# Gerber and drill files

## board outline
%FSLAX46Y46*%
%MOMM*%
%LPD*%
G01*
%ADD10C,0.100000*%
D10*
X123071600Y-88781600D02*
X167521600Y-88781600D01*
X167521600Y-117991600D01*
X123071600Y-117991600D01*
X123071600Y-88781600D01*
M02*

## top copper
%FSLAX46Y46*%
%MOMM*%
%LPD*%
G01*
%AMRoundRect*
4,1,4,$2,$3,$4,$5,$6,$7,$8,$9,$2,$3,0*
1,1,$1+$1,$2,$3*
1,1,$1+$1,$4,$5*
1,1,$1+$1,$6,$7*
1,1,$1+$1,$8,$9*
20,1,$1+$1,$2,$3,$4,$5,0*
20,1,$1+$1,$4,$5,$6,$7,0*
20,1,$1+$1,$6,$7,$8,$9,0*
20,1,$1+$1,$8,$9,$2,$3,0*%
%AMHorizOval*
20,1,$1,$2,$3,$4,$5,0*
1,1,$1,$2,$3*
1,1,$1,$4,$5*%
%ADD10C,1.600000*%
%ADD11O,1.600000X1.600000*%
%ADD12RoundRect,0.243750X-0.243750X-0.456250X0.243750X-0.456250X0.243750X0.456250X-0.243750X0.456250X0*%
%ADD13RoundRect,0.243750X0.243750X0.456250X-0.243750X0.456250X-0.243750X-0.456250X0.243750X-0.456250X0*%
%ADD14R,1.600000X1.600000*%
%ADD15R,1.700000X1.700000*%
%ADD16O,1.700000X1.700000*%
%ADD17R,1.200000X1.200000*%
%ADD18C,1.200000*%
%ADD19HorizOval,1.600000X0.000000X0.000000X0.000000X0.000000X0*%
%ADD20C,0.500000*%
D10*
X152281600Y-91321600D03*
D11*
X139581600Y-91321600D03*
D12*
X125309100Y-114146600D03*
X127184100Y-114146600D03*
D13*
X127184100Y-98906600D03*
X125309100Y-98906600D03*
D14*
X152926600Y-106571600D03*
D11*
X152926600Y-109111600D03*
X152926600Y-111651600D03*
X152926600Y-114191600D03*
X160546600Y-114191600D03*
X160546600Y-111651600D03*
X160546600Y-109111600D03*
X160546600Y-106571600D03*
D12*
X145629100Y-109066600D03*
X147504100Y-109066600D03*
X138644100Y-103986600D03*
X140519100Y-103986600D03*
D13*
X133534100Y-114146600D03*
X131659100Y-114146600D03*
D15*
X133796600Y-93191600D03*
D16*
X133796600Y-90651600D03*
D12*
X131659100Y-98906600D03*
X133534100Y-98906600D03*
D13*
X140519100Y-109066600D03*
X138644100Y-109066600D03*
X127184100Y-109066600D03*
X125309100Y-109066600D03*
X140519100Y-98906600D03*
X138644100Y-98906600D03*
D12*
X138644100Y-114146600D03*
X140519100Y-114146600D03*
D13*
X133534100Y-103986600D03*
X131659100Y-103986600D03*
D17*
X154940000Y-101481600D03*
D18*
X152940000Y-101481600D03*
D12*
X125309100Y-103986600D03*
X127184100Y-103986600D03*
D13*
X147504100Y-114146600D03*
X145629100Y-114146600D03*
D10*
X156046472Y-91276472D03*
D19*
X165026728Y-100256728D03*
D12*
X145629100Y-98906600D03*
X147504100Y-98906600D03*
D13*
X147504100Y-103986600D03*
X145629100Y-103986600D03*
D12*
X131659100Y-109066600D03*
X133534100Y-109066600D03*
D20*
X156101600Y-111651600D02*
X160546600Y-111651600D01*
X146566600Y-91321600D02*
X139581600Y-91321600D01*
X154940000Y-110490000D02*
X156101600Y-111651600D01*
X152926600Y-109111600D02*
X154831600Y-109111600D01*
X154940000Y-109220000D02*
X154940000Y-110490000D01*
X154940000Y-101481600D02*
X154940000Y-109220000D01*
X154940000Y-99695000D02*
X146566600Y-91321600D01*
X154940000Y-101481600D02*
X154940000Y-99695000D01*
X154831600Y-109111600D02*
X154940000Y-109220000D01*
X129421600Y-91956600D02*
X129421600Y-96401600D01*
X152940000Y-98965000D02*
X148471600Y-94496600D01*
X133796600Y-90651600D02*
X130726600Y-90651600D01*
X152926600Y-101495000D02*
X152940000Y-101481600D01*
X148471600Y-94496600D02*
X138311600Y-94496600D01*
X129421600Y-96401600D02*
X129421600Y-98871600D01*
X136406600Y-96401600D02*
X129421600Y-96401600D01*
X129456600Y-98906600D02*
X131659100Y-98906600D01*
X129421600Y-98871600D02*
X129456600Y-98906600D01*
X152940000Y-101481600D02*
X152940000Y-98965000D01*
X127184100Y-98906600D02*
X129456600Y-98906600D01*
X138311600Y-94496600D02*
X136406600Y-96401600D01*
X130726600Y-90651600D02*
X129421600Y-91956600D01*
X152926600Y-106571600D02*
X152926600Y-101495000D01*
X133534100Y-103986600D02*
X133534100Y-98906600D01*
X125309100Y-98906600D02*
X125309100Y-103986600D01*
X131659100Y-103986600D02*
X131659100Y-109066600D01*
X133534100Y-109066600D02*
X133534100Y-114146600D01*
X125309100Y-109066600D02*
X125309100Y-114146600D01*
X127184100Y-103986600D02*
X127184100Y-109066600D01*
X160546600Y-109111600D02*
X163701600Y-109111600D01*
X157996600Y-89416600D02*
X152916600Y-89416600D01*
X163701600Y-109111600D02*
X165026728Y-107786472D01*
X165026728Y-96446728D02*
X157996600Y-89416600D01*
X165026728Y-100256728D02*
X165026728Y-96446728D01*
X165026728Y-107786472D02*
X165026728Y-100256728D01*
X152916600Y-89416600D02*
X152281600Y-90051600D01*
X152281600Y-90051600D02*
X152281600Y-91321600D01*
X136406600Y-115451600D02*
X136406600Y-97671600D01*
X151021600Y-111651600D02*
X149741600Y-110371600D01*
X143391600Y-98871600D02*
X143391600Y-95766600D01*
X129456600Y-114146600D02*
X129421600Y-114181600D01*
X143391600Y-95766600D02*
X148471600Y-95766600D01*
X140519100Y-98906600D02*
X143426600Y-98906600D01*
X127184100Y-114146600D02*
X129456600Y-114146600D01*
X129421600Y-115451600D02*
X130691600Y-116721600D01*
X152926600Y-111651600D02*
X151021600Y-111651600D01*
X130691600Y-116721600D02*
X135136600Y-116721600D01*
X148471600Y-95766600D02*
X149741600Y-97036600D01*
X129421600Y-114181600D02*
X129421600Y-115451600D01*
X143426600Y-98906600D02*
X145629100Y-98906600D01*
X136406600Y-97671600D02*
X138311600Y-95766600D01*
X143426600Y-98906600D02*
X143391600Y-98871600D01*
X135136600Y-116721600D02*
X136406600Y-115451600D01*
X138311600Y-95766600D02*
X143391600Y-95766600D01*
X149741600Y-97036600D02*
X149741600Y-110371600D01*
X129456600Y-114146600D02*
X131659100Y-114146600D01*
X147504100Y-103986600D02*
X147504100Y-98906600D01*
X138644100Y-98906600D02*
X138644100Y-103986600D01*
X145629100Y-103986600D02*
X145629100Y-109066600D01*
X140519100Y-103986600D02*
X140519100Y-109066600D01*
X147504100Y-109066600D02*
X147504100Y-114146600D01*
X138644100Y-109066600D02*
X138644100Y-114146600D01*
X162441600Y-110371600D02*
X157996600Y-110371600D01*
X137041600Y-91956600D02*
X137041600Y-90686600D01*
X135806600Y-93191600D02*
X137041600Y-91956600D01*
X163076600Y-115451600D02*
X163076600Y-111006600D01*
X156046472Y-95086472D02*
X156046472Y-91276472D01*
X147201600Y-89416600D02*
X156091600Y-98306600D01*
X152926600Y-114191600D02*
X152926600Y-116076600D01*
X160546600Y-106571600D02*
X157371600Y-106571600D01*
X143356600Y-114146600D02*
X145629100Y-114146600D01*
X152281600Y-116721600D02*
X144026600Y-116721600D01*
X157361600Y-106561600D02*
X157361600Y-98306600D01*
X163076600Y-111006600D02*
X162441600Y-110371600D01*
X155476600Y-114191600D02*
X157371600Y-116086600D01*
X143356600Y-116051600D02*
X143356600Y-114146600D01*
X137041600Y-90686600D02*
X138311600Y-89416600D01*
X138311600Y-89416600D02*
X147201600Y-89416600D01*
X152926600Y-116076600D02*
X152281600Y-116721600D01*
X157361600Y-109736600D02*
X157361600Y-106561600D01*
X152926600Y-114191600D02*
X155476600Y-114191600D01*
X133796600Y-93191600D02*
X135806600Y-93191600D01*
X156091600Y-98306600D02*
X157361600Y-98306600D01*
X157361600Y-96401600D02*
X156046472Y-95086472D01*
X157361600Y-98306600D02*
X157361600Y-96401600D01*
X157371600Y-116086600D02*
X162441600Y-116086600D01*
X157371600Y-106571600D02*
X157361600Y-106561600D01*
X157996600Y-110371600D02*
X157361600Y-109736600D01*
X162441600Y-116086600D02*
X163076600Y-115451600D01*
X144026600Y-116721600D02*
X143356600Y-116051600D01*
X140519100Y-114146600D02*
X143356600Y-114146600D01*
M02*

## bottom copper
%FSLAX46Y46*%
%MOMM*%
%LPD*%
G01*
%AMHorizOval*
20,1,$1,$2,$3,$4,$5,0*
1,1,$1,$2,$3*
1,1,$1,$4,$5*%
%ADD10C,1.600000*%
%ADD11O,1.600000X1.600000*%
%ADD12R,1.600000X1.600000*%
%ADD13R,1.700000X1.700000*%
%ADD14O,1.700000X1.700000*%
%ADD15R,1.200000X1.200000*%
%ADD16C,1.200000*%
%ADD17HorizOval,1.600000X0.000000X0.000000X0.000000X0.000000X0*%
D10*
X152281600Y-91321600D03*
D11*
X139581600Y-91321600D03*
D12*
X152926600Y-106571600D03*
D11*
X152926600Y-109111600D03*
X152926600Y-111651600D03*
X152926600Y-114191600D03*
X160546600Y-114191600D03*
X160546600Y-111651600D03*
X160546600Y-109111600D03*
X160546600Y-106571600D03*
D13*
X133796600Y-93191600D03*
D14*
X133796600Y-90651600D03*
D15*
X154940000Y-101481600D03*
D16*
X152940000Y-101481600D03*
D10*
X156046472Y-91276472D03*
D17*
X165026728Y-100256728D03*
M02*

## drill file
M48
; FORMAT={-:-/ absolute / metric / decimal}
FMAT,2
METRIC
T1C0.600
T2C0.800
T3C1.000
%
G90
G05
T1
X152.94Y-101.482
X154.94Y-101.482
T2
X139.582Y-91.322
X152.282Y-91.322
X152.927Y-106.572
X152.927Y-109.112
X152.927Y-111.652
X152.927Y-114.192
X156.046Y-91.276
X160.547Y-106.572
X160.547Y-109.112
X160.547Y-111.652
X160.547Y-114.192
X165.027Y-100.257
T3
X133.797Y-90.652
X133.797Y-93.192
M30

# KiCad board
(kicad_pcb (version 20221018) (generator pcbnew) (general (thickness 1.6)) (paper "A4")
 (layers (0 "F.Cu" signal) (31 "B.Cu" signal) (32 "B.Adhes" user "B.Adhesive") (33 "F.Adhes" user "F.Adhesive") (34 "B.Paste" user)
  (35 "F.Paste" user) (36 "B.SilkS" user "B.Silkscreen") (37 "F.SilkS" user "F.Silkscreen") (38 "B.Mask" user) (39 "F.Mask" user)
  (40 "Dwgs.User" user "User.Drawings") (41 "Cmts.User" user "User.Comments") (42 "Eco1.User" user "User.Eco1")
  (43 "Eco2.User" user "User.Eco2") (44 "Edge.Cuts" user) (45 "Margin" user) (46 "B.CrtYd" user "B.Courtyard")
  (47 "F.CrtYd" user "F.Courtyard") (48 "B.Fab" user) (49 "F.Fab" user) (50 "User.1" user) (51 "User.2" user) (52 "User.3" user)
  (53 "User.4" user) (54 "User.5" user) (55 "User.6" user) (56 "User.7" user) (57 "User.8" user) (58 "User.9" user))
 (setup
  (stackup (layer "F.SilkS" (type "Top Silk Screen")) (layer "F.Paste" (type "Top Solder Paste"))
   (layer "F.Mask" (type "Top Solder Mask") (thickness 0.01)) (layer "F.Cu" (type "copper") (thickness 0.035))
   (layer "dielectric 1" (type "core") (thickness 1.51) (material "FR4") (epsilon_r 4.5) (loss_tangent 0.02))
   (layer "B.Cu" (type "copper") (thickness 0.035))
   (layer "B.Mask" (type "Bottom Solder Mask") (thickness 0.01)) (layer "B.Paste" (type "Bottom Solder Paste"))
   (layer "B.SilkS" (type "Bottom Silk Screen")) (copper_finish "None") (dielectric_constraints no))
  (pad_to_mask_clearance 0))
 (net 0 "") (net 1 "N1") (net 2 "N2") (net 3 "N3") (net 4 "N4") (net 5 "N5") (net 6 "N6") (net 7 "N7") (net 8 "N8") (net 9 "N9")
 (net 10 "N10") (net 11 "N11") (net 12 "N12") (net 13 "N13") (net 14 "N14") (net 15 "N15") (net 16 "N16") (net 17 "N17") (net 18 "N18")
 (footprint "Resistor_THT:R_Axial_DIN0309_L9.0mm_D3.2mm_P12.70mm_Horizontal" (layer "F.Cu") (at 152.2816 91.3216 180)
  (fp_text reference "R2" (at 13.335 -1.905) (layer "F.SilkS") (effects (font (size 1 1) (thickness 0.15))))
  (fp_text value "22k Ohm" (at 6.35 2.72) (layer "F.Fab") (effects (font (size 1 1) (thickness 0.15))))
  (pad "1" thru_hole circle (at 0 0 180) (size 1.6 1.6) (drill 0.8) (layers "*.Cu" "*.Mask") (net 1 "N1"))
  (pad "2" thru_hole oval (at 12.7 0 180) (size 1.6 1.6) (drill 0.8) (layers "*.Cu" "*.Mask") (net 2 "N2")))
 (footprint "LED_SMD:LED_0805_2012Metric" (layer "F.Cu") (at 126.2466 114.1466)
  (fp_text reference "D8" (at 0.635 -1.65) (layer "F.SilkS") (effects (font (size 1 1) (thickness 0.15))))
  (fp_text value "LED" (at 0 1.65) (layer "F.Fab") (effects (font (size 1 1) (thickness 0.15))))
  (pad "1" smd roundrect (at -0.9375 0) (size 0.975 1.4) (layers "F.Cu" "F.Paste" "F.Mask") (roundrect_rratio 0.25) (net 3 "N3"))
  (pad "2" smd roundrect (at 0.9375 0) (size 0.975 1.4) (layers "F.Cu" "F.Paste" "F.Mask") (roundrect_rratio 0.25) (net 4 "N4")))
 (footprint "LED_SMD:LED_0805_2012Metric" (layer "F.Cu") (at 126.2466 98.9066 180)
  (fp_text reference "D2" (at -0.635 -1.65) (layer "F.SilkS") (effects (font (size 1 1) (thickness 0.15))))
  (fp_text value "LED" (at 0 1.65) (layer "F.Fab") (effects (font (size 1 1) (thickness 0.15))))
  (pad "1" smd roundrect (at -0.9375 0 180) (size 0.975 1.4) (layers "F.Cu" "F.Paste" "F.Mask") (roundrect_rratio 0.25) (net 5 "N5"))
  (pad "2" smd roundrect (at 0.9375 0 180) (size 0.975 1.4) (layers "F.Cu" "F.Paste" "F.Mask") (roundrect_rratio 0.25) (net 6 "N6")))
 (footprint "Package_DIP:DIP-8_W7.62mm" (layer "F.Cu") (at 152.9266 106.5716)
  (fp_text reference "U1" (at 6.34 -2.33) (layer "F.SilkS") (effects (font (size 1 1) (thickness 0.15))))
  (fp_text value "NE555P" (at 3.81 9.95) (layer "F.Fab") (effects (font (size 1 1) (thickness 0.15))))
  (pad "1" thru_hole rect (at 0 0) (size 1.6 1.6) (drill 0.8) (layers "*.Cu" "*.Mask") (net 5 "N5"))
  (pad "2" thru_hole oval (at 0 2.54) (size 1.6 1.6) (drill 0.8) (layers "*.Cu" "*.Mask") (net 2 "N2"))
  (pad "3" thru_hole oval (at 0 5.08) (size 1.6 1.6) (drill 0.8) (layers "*.Cu" "*.Mask") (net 4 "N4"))
  (pad "4" thru_hole oval (at 0 7.62) (size 1.6 1.6) (drill 0.8) (layers "*.Cu" "*.Mask") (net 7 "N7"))
  (pad "5" thru_hole oval (at 7.62 7.62) (size 1.6 1.6) (drill 0.8) (layers "*.Cu" "*.Mask") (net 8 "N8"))
  (pad "6" thru_hole oval (at 7.62 5.08) (size 1.6 1.6) (drill 0.8) (layers "*.Cu" "*.Mask") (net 2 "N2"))
  (pad "7" thru_hole oval (at 7.62 2.54) (size 1.6 1.6) (drill 0.8) (layers "*.Cu" "*.Mask") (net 1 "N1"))
  (pad "8" thru_hole oval (at 7.62 0) (size 1.6 1.6) (drill 0.8) (layers "*.Cu" "*.Mask") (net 7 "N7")))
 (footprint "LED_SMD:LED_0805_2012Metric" (layer "F.Cu") (at 146.5666 109.0666)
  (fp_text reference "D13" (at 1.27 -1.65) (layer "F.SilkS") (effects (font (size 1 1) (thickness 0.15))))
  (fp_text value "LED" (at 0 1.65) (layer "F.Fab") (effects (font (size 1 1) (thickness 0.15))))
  (pad "1" smd roundrect (at -0.9375 0) (size 0.975 1.4) (layers "F.Cu" "F.Paste" "F.Mask") (roundrect_rratio 0.25) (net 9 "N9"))
  (pad "2" smd roundrect (at 0.9375 0) (size 0.975 1.4) (layers "F.Cu" "F.Paste" "F.Mask") (roundrect_rratio 0.25) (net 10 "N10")))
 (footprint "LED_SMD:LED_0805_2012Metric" (layer "F.Cu") (at 139.5816 103.9866)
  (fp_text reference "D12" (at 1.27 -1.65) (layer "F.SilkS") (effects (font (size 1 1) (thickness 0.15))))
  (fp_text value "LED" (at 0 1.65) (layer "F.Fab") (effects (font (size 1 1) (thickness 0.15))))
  (pad "1" smd roundrect (at -0.9375 0) (size 0.975 1.4) (layers "F.Cu" "F.Paste" "F.Mask") (roundrect_rratio 0.25) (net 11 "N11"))
  (pad "2" smd roundrect (at 0.9375 0) (size 0.975 1.4) (layers "F.Cu" "F.Paste" "F.Mask") (roundrect_rratio 0.25) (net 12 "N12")))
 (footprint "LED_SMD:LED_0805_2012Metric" (layer "F.Cu") (at 132.5966 114.1466 180)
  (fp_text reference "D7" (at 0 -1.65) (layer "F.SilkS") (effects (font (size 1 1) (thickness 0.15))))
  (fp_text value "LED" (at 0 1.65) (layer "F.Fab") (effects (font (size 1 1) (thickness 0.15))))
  (pad "1" smd roundrect (at -0.9375 0 180) (size 0.975 1.4) (layers "F.Cu" "F.Paste" "F.Mask") (roundrect_rratio 0.25) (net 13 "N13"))
  (pad "2" smd roundrect (at 0.9375 0 180) (size 0.975 1.4) (layers "F.Cu" "F.Paste" "F.Mask") (roundrect_rratio 0.25) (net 4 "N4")))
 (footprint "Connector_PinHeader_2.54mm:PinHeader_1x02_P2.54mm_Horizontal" (layer "F.Cu") (at 133.7966 93.1916 180)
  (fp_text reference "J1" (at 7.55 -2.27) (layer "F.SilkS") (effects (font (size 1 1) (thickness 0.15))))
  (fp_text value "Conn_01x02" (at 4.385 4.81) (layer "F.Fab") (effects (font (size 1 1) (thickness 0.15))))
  (pad "1" thru_hole rect (at 0 0 180) (size 1.7 1.7) (drill 1) (layers "*.Cu" "*.Mask") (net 7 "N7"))
  (pad "2" thru_hole oval (at 0 2.54 180) (size 1.7 1.7) (drill 1) (layers "*.Cu" "*.Mask") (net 5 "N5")))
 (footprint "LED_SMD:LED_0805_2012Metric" (layer "F.Cu") (at 132.5966 98.9066)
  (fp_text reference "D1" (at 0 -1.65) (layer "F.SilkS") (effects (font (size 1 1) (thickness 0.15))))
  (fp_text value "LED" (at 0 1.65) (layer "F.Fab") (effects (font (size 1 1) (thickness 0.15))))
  (pad "1" smd roundrect (at -0.9375 0) (size 0.975 1.4) (layers "F.Cu" "F.Paste" "F.Mask") (roundrect_rratio 0.25) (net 5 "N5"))
  (pad "2" smd roundrect (at 0.9375 0) (size 0.975 1.4) (layers "F.Cu" "F.Paste" "F.Mask") (roundrect_rratio 0.25) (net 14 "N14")))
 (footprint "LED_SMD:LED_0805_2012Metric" (layer "F.Cu") (at 139.5816 109.0666 180)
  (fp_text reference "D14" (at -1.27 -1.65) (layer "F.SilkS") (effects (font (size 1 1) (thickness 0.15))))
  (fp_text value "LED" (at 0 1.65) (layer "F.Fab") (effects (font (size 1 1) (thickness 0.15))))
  (pad "1" smd roundrect (at -0.9375 0 180) (size 0.975 1.4) (layers "F.Cu" "F.Paste" "F.Mask") (roundrect_rratio 0.25) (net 12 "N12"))
  (pad "2" smd roundrect (at 0.9375 0 180) (size 0.975 1.4) (layers "F.Cu" "F.Paste" "F.Mask") (roundrect_rratio 0.25) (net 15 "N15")))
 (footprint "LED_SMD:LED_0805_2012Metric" (layer "F.Cu") (at 126.2466 109.0666 180)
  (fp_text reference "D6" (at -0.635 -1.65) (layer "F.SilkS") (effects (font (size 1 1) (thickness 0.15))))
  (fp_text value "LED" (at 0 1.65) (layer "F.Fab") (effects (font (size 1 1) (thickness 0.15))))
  (pad "1" smd roundrect (at -0.9375 0 180) (size 0.975 1.4) (layers "F.Cu" "F.Paste" "F.Mask") (roundrect_rratio 0.25) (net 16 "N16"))
  (pad "2" smd roundrect (at 0.9375 0 180) (size 0.975 1.4) (layers "F.Cu" "F.Paste" "F.Mask") (roundrect_rratio 0.25) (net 3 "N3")))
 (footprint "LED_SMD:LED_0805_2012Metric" (layer "F.Cu") (at 139.5816 98.9066 180)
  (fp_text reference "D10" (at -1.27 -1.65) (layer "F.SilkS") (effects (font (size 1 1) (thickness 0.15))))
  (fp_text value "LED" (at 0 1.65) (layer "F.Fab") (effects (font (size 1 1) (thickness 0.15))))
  (pad "1" smd roundrect (at -0.9375 0 180) (size 0.975 1.4) (layers "F.Cu" "F.Paste" "F.Mask") (roundrect_rratio 0.25) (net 4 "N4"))
  (pad "2" smd roundrect (at 0.9375 0 180) (size 0.975 1.4) (layers "F.Cu" "F.Paste" "F.Mask") (roundrect_rratio 0.25) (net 11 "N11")))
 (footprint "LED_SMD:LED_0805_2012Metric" (layer "F.Cu") (at 139.5816 114.1466)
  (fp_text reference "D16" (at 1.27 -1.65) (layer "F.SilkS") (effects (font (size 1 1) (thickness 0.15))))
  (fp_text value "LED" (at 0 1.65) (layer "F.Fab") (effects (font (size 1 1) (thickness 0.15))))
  (pad "1" smd roundrect (at -0.9375 0) (size 0.975 1.4) (layers "F.Cu" "F.Paste" "F.Mask") (roundrect_rratio 0.25) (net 15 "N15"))
  (pad "2" smd roundrect (at 0.9375 0) (size 0.975 1.4) (layers "F.Cu" "F.Paste" "F.Mask") (roundrect_rratio 0.25) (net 7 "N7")))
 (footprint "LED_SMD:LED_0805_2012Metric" (layer "F.Cu") (at 132.5966 103.9866 180)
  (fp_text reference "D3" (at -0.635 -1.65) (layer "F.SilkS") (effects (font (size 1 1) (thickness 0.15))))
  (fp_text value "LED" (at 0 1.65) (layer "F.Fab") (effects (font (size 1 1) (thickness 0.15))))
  (pad "1" smd roundrect (at -0.9375 0 180) (size 0.975 1.4) (layers "F.Cu" "F.Paste" "F.Mask") (roundrect_rratio 0.25) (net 14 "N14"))
  (pad "2" smd roundrect (at 0.9375 0 180) (size 0.975 1.4) (layers "F.Cu" "F.Paste" "F.Mask") (roundrect_rratio 0.25) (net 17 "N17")))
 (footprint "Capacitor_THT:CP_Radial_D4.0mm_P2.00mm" (layer "F.Cu") (at 154.94 101.4816 180)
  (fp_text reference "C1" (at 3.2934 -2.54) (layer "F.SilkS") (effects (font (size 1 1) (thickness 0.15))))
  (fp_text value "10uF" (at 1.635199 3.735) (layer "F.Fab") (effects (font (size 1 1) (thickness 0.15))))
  (pad "1" thru_hole rect (at 0 0 180) (size 1.2 1.2) (drill 0.6) (layers "*.Cu" "*.Mask") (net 2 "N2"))
  (pad "2" thru_hole circle (at 2 0 180) (size 1.2 1.2) (drill 0.6) (layers "*.Cu" "*.Mask") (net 5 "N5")))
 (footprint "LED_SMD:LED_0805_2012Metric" (layer "F.Cu") (at 126.2466 103.9866)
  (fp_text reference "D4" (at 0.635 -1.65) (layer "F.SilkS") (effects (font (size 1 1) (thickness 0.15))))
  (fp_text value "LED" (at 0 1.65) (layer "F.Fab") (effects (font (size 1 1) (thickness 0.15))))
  (pad "1" smd roundrect (at -0.9375 0) (size 0.975 1.4) (layers "F.Cu" "F.Paste" "F.Mask") (roundrect_rratio 0.25) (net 6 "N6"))
  (pad "2" smd roundrect (at 0.9375 0) (size 0.975 1.4) (layers "F.Cu" "F.Paste" "F.Mask") (roundrect_rratio 0.25) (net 16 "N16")))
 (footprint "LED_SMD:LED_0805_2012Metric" (layer "F.Cu") (at 146.5666 114.1466 180)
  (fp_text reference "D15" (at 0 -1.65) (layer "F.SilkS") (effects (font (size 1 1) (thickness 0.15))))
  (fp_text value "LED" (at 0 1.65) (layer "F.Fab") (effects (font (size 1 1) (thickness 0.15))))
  (pad "1" smd roundrect (at -0.9375 0 180) (size 0.975 1.4) (layers "F.Cu" "F.Paste" "F.Mask") (roundrect_rratio 0.25) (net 10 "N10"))
  (pad "2" smd roundrect (at 0.9375 0 180) (size 0.975 1.4) (layers "F.Cu" "F.Paste" "F.Mask") (roundrect_rratio 0.25) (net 7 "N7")))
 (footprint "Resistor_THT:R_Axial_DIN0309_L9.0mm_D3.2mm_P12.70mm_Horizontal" (layer "F.Cu") (at 156.046472 91.276472 -45)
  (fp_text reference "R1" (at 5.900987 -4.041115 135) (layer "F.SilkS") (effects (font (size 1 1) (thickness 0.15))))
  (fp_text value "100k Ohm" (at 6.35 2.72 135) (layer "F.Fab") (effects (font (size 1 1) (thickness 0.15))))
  (pad "1" thru_hole circle (at 0 0 315) (size 1.6 1.6) (drill 0.8) (layers "*.Cu" "*.Mask") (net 7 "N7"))
  (pad "2" thru_hole oval (at 12.7 0 315) (size 1.6 1.6) (drill 0.8) (layers "*.Cu" "*.Mask") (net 1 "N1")))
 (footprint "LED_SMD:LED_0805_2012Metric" (layer "F.Cu") (at 146.5666 98.9066)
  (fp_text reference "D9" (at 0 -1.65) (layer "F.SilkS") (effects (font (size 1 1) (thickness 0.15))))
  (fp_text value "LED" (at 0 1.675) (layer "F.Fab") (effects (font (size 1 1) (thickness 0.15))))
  (pad "1" smd roundrect (at -0.9375 0) (size 0.975 1.4) (layers "F.Cu" "F.Paste" "F.Mask") (roundrect_rratio 0.25) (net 4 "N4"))
  (pad "2" smd roundrect (at 0.9375 0) (size 0.975 1.4) (layers "F.Cu" "F.Paste" "F.Mask") (roundrect_rratio 0.25) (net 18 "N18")))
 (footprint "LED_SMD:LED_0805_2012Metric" (layer "F.Cu") (at 146.5666 103.9866 180)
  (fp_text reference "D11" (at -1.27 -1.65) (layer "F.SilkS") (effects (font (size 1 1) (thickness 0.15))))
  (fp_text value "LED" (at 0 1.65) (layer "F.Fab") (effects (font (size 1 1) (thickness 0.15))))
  (pad "1" smd roundrect (at -0.9375 0 180) (size 0.975 1.4) (layers "F.Cu" "F.Paste" "F.Mask") (roundrect_rratio 0.25) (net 18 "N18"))
  (pad "2" smd roundrect (at 0.9375 0 180) (size 0.975 1.4) (layers "F.Cu" "F.Paste" "F.Mask") (roundrect_rratio 0.25) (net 9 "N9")))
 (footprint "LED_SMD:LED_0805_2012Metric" (layer "F.Cu") (at 132.5966 109.0666)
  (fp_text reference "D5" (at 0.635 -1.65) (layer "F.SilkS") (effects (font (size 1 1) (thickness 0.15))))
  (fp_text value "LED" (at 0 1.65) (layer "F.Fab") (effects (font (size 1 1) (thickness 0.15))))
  (pad "1" smd roundrect (at -0.9375 0) (size 0.975 1.4) (layers "F.Cu" "F.Paste" "F.Mask") (roundrect_rratio 0.25) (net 17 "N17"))
  (pad "2" smd roundrect (at 0.9375 0) (size 0.975 1.4) (layers "F.Cu" "F.Paste" "F.Mask") (roundrect_rratio 0.25) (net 13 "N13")))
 (gr_rect (start 123.0716 88.7816) (end 167.5216 117.9916) (stroke (width 0.1) (type solid)) (fill none) (layer "Edge.Cuts"))
 (segment (start 156.1016 111.6516) (end 160.5466 111.6516) (width 0.5) (layer "F.Cu") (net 2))
 (segment (start 146.5666 91.3216) (end 139.5816 91.3216) (width 0.5) (layer "F.Cu") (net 2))
 (segment (start 154.94 110.49) (end 156.1016 111.6516) (width 0.5) (layer "F.Cu") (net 2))
 (segment (start 152.9266 109.1116) (end 154.8316 109.1116) (width 0.5) (layer "F.Cu") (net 2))
 (segment (start 154.94 109.22) (end 154.94 110.49) (width 0.5) (layer "F.Cu") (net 2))
 (segment (start 154.94 101.4816) (end 154.94 109.22) (width 0.5) (layer "F.Cu") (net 2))
 (segment (start 154.94 99.695) (end 146.5666 91.3216) (width 0.5) (layer "F.Cu") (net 2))
 (segment (start 154.94 101.4816) (end 154.94 99.695) (width 0.5) (layer "F.Cu") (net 2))
 (segment (start 154.8316 109.1116) (end 154.94 109.22) (width 0.5) (layer "F.Cu") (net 2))
 (segment (start 129.4216 91.9566) (end 129.4216 96.4016) (width 0.5) (layer "F.Cu") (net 5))
 (segment (start 152.94 98.965) (end 148.4716 94.4966) (width 0.5) (layer "F.Cu") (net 5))
 (segment (start 133.7966 90.6516) (end 130.7266 90.6516) (width 0.5) (layer "F.Cu") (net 5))
 (segment (start 152.9266 101.495) (end 152.94 101.4816) (width 0.5) (layer "F.Cu") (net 5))
 (segment (start 148.4716 94.4966) (end 138.3116 94.4966) (width 0.5) (layer "F.Cu") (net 5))
 (segment (start 129.4216 96.4016) (end 129.4216 98.8716) (width 0.5) (layer "F.Cu") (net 5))
 (segment (start 136.4066 96.4016) (end 129.4216 96.4016) (width 0.5) (layer "F.Cu") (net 5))
 (segment (start 129.4566 98.9066) (end 131.6591 98.9066) (width 0.5) (layer "F.Cu") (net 5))
 (segment (start 129.4216 98.8716) (end 129.4566 98.9066) (width 0.5) (layer "F.Cu") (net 5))
 (segment (start 152.94 101.4816) (end 152.94 98.965) (width 0.5) (layer "F.Cu") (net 5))
 (segment (start 127.1841 98.9066) (end 129.4566 98.9066) (width 0.5) (layer "F.Cu") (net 5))
 (segment (start 138.3116 94.4966) (end 136.4066 96.4016) (width 0.5) (layer "F.Cu") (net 5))
 (segment (start 130.7266 90.6516) (end 129.4216 91.9566) (width 0.5) (layer "F.Cu") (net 5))
 (segment (start 152.9266 106.5716) (end 152.9266 101.495) (width 0.5) (layer "F.Cu") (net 5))
 (segment (start 133.5341 103.9866) (end 133.5341 98.9066) (width 0.5) (layer "F.Cu") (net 14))
 (segment (start 125.3091 98.9066) (end 125.3091 103.9866) (width 0.5) (layer "F.Cu") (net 6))
 (segment (start 131.6591 103.9866) (end 131.6591 109.0666) (width 0.5) (layer "F.Cu") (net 17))
 (segment (start 133.5341 109.0666) (end 133.5341 114.1466) (width 0.5) (layer "F.Cu") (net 13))
 (segment (start 125.3091 109.0666) (end 125.3091 114.1466) (width 0.5) (layer "F.Cu") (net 3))
 (segment (start 127.1841 103.9866) (end 127.1841 109.0666) (width 0.5) (layer "F.Cu") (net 16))
 (segment (start 160.5466 109.1116) (end 163.7016 109.1116) (width 0.5) (layer "F.Cu") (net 1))
 (segment (start 157.9966 89.4166) (end 152.9166 89.4166) (width 0.5) (layer "F.Cu") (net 1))
 (segment (start 163.7016 109.1116) (end 165.026728 107.786472) (width 0.5) (layer "F.Cu") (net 1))
 (segment (start 165.026728 96.446728) (end 157.9966 89.4166) (width 0.5) (layer "F.Cu") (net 1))
 (segment (start 165.026728 100.256728) (end 165.026728 96.446728) (width 0.5) (layer "F.Cu") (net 1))
 (segment (start 165.026728 107.786472) (end 165.026728 100.256728) (width 0.5) (layer "F.Cu") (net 1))
 (segment (start 152.9166 89.4166) (end 152.2816 90.0516) (width 0.5) (layer "F.Cu") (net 1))
 (segment (start 152.2816 90.0516) (end 152.2816 91.3216) (width 0.5) (layer "F.Cu") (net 1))
 (segment (start 136.4066 115.4516) (end 136.4066 97.6716) (width 0.5) (layer "F.Cu") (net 4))
 (segment (start 151.0216 111.6516) (end 149.7416 110.3716) (width 0.5) (layer "F.Cu") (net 4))
 (segment (start 143.3916 98.8716) (end 143.3916 95.7666) (width 0.5) (layer "F.Cu") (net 4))
 (segment (start 129.4566 114.1466) (end 129.4216 114.1816) (width 0.5) (layer "F.Cu") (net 4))
 (segment (start 143.3916 95.7666) (end 148.4716 95.7666) (width 0.5) (layer "F.Cu") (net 4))
 (segment (start 140.5191 98.9066) (end 143.4266 98.9066) (width 0.5) (layer "F.Cu") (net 4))
 (segment (start 127.1841 114.1466) (end 129.4566 114.1466) (width 0.5) (layer "F.Cu") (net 4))
 (segment (start 129.4216 115.4516) (end 130.6916 116.7216) (width 0.5) (layer "F.Cu") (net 4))
 (segment (start 152.9266 111.6516) (end 151.0216 111.6516) (width 0.5) (layer "F.Cu") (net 4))
 (segment (start 130.6916 116.7216) (end 135.1366 116.7216) (width 0.5) (layer "F.Cu") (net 4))
 (segment (start 148.4716 95.7666) (end 149.7416 97.0366) (width 0.5) (layer "F.Cu") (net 4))
 (segment (start 129.4216 114.1816) (end 129.4216 115.4516) (width 0.5) (layer "F.Cu") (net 4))
 (segment (start 143.4266 98.9066) (end 145.6291 98.9066) (width 0.5) (layer "F.Cu") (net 4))
 (segment (start 136.4066 97.6716) (end 138.3116 95.7666) (width 0.5) (layer "F.Cu") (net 4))
 (segment (start 143.4266 98.9066) (end 143.3916 98.8716) (width 0.5) (layer "F.Cu") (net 4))
 (segment (start 135.1366 116.7216) (end 136.4066 115.4516) (width 0.5) (layer "F.Cu") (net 4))
 (segment (start 138.3116 95.7666) (end 143.3916 95.7666) (width 0.5) (layer "F.Cu") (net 4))
 (segment (start 149.7416 97.0366) (end 149.7416 110.3716) (width 0.5) (layer "F.Cu") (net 4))
 (segment (start 129.4566 114.1466) (end 131.6591 114.1466) (width 0.5) (layer "F.Cu") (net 4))
 (segment (start 147.5041 103.9866) (end 147.5041 98.9066) (width 0.5) (layer "F.Cu") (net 18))
 (segment (start 138.6441 98.9066) (end 138.6441 103.9866) (width 0.5) (layer "F.Cu") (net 11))
 (segment (start 145.6291 103.9866) (end 145.6291 109.0666) (width 0.5) (layer "F.Cu") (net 9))
 (segment (start 140.5191 103.9866) (end 140.5191 109.0666) (width 0.5) (layer "F.Cu") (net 12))
 (segment (start 147.5041 109.0666) (end 147.5041 114.1466) (width 0.5) (layer "F.Cu") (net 10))
 (segment (start 138.6441 109.0666) (end 138.6441 114.1466) (width 0.5) (layer "F.Cu") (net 15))
 (segment (start 162.4416 110.3716) (end 157.9966 110.3716) (width 0.5) (layer "F.Cu") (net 7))
 (segment (start 137.0416 91.9566) (end 137.0416 90.6866) (width 0.5) (layer "F.Cu") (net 7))
 (segment (start 135.8066 93.1916) (end 137.0416 91.9566) (width 0.5) (layer "F.Cu") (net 7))
 (segment (start 163.0766 115.4516) (end 163.0766 111.0066) (width 0.5) (layer "F.Cu") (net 7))
 (segment (start 156.046472 95.086472) (end 156.046472 91.276472) (width 0.5) (layer "F.Cu") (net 7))
 (segment (start 147.2016 89.4166) (end 156.0916 98.3066) (width 0.5) (layer "F.Cu") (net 7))
 (segment (start 152.9266 114.1916) (end 152.9266 116.0766) (width 0.5) (layer "F.Cu") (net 7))
 (segment (start 160.5466 106.5716) (end 157.3716 106.5716) (width 0.5) (layer "F.Cu") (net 7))
 (segment (start 143.3566 114.1466) (end 145.6291 114.1466) (width 0.5) (layer "F.Cu") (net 7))
 (segment (start 152.2816 116.7216) (end 144.0266 116.7216) (width 0.5) (layer "F.Cu") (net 7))
 (segment (start 157.3616 106.5616) (end 157.3616 98.3066) (width 0.5) (layer "F.Cu") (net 7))
 (segment (start 163.0766 111.0066) (end 162.4416 110.3716) (width 0.5) (layer "F.Cu") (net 7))
 (segment (start 155.4766 114.1916) (end 157.3716 116.0866) (width 0.5) (layer "F.Cu") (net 7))
 (segment (start 143.3566 116.0516) (end 143.3566 114.1466) (width 0.5) (layer "F.Cu") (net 7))
 (segment (start 137.0416 90.6866) (end 138.3116 89.4166) (width 0.5) (layer "F.Cu") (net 7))
 (segment (start 138.3116 89.4166) (end 147.2016 89.4166) (width 0.5) (layer "F.Cu") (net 7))
 (segment (start 152.9266 116.0766) (end 152.2816 116.7216) (width 0.5) (layer "F.Cu") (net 7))
 (segment (start 157.3616 109.7366) (end 157.3616 106.5616) (width 0.5) (layer "F.Cu") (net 7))
 (segment (start 152.9266 114.1916) (end 155.4766 114.1916) (width 0.5) (layer "F.Cu") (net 7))
 (segment (start 133.7966 93.1916) (end 135.8066 93.1916) (width 0.5) (layer "F.Cu") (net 7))
 (segment (start 156.0916 98.3066) (end 157.3616 98.3066) (width 0.5) (layer "F.Cu") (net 7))
 (segment (start 157.3616 96.4016) (end 156.046472 95.086472) (width 0.5) (layer "F.Cu") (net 7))
 (segment (start 157.3616 98.3066) (end 157.3616 96.4016) (width 0.5) (layer "F.Cu") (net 7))
 (segment (start 157.3716 116.0866) (end 162.4416 116.0866) (width 0.5) (layer "F.Cu") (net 7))
 (segment (start 157.3716 106.5716) (end 157.3616 106.5616) (width 0.5) (layer "F.Cu") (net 7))
 (segment (start 157.9966 110.3716) (end 157.3616 109.7366) (width 0.5) (layer "F.Cu") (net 7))
 (segment (start 162.4416 116.0866) (end 163.0766 115.4516) (width 0.5) (layer "F.Cu") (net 7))
 (segment (start 144.0266 116.7216) (end 143.3566 116.0516) (width 0.5) (layer "F.Cu") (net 7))
 (segment (start 140.5191 114.1466) (end 143.3566 114.1466) (width 0.5) (layer "F.Cu") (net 7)))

